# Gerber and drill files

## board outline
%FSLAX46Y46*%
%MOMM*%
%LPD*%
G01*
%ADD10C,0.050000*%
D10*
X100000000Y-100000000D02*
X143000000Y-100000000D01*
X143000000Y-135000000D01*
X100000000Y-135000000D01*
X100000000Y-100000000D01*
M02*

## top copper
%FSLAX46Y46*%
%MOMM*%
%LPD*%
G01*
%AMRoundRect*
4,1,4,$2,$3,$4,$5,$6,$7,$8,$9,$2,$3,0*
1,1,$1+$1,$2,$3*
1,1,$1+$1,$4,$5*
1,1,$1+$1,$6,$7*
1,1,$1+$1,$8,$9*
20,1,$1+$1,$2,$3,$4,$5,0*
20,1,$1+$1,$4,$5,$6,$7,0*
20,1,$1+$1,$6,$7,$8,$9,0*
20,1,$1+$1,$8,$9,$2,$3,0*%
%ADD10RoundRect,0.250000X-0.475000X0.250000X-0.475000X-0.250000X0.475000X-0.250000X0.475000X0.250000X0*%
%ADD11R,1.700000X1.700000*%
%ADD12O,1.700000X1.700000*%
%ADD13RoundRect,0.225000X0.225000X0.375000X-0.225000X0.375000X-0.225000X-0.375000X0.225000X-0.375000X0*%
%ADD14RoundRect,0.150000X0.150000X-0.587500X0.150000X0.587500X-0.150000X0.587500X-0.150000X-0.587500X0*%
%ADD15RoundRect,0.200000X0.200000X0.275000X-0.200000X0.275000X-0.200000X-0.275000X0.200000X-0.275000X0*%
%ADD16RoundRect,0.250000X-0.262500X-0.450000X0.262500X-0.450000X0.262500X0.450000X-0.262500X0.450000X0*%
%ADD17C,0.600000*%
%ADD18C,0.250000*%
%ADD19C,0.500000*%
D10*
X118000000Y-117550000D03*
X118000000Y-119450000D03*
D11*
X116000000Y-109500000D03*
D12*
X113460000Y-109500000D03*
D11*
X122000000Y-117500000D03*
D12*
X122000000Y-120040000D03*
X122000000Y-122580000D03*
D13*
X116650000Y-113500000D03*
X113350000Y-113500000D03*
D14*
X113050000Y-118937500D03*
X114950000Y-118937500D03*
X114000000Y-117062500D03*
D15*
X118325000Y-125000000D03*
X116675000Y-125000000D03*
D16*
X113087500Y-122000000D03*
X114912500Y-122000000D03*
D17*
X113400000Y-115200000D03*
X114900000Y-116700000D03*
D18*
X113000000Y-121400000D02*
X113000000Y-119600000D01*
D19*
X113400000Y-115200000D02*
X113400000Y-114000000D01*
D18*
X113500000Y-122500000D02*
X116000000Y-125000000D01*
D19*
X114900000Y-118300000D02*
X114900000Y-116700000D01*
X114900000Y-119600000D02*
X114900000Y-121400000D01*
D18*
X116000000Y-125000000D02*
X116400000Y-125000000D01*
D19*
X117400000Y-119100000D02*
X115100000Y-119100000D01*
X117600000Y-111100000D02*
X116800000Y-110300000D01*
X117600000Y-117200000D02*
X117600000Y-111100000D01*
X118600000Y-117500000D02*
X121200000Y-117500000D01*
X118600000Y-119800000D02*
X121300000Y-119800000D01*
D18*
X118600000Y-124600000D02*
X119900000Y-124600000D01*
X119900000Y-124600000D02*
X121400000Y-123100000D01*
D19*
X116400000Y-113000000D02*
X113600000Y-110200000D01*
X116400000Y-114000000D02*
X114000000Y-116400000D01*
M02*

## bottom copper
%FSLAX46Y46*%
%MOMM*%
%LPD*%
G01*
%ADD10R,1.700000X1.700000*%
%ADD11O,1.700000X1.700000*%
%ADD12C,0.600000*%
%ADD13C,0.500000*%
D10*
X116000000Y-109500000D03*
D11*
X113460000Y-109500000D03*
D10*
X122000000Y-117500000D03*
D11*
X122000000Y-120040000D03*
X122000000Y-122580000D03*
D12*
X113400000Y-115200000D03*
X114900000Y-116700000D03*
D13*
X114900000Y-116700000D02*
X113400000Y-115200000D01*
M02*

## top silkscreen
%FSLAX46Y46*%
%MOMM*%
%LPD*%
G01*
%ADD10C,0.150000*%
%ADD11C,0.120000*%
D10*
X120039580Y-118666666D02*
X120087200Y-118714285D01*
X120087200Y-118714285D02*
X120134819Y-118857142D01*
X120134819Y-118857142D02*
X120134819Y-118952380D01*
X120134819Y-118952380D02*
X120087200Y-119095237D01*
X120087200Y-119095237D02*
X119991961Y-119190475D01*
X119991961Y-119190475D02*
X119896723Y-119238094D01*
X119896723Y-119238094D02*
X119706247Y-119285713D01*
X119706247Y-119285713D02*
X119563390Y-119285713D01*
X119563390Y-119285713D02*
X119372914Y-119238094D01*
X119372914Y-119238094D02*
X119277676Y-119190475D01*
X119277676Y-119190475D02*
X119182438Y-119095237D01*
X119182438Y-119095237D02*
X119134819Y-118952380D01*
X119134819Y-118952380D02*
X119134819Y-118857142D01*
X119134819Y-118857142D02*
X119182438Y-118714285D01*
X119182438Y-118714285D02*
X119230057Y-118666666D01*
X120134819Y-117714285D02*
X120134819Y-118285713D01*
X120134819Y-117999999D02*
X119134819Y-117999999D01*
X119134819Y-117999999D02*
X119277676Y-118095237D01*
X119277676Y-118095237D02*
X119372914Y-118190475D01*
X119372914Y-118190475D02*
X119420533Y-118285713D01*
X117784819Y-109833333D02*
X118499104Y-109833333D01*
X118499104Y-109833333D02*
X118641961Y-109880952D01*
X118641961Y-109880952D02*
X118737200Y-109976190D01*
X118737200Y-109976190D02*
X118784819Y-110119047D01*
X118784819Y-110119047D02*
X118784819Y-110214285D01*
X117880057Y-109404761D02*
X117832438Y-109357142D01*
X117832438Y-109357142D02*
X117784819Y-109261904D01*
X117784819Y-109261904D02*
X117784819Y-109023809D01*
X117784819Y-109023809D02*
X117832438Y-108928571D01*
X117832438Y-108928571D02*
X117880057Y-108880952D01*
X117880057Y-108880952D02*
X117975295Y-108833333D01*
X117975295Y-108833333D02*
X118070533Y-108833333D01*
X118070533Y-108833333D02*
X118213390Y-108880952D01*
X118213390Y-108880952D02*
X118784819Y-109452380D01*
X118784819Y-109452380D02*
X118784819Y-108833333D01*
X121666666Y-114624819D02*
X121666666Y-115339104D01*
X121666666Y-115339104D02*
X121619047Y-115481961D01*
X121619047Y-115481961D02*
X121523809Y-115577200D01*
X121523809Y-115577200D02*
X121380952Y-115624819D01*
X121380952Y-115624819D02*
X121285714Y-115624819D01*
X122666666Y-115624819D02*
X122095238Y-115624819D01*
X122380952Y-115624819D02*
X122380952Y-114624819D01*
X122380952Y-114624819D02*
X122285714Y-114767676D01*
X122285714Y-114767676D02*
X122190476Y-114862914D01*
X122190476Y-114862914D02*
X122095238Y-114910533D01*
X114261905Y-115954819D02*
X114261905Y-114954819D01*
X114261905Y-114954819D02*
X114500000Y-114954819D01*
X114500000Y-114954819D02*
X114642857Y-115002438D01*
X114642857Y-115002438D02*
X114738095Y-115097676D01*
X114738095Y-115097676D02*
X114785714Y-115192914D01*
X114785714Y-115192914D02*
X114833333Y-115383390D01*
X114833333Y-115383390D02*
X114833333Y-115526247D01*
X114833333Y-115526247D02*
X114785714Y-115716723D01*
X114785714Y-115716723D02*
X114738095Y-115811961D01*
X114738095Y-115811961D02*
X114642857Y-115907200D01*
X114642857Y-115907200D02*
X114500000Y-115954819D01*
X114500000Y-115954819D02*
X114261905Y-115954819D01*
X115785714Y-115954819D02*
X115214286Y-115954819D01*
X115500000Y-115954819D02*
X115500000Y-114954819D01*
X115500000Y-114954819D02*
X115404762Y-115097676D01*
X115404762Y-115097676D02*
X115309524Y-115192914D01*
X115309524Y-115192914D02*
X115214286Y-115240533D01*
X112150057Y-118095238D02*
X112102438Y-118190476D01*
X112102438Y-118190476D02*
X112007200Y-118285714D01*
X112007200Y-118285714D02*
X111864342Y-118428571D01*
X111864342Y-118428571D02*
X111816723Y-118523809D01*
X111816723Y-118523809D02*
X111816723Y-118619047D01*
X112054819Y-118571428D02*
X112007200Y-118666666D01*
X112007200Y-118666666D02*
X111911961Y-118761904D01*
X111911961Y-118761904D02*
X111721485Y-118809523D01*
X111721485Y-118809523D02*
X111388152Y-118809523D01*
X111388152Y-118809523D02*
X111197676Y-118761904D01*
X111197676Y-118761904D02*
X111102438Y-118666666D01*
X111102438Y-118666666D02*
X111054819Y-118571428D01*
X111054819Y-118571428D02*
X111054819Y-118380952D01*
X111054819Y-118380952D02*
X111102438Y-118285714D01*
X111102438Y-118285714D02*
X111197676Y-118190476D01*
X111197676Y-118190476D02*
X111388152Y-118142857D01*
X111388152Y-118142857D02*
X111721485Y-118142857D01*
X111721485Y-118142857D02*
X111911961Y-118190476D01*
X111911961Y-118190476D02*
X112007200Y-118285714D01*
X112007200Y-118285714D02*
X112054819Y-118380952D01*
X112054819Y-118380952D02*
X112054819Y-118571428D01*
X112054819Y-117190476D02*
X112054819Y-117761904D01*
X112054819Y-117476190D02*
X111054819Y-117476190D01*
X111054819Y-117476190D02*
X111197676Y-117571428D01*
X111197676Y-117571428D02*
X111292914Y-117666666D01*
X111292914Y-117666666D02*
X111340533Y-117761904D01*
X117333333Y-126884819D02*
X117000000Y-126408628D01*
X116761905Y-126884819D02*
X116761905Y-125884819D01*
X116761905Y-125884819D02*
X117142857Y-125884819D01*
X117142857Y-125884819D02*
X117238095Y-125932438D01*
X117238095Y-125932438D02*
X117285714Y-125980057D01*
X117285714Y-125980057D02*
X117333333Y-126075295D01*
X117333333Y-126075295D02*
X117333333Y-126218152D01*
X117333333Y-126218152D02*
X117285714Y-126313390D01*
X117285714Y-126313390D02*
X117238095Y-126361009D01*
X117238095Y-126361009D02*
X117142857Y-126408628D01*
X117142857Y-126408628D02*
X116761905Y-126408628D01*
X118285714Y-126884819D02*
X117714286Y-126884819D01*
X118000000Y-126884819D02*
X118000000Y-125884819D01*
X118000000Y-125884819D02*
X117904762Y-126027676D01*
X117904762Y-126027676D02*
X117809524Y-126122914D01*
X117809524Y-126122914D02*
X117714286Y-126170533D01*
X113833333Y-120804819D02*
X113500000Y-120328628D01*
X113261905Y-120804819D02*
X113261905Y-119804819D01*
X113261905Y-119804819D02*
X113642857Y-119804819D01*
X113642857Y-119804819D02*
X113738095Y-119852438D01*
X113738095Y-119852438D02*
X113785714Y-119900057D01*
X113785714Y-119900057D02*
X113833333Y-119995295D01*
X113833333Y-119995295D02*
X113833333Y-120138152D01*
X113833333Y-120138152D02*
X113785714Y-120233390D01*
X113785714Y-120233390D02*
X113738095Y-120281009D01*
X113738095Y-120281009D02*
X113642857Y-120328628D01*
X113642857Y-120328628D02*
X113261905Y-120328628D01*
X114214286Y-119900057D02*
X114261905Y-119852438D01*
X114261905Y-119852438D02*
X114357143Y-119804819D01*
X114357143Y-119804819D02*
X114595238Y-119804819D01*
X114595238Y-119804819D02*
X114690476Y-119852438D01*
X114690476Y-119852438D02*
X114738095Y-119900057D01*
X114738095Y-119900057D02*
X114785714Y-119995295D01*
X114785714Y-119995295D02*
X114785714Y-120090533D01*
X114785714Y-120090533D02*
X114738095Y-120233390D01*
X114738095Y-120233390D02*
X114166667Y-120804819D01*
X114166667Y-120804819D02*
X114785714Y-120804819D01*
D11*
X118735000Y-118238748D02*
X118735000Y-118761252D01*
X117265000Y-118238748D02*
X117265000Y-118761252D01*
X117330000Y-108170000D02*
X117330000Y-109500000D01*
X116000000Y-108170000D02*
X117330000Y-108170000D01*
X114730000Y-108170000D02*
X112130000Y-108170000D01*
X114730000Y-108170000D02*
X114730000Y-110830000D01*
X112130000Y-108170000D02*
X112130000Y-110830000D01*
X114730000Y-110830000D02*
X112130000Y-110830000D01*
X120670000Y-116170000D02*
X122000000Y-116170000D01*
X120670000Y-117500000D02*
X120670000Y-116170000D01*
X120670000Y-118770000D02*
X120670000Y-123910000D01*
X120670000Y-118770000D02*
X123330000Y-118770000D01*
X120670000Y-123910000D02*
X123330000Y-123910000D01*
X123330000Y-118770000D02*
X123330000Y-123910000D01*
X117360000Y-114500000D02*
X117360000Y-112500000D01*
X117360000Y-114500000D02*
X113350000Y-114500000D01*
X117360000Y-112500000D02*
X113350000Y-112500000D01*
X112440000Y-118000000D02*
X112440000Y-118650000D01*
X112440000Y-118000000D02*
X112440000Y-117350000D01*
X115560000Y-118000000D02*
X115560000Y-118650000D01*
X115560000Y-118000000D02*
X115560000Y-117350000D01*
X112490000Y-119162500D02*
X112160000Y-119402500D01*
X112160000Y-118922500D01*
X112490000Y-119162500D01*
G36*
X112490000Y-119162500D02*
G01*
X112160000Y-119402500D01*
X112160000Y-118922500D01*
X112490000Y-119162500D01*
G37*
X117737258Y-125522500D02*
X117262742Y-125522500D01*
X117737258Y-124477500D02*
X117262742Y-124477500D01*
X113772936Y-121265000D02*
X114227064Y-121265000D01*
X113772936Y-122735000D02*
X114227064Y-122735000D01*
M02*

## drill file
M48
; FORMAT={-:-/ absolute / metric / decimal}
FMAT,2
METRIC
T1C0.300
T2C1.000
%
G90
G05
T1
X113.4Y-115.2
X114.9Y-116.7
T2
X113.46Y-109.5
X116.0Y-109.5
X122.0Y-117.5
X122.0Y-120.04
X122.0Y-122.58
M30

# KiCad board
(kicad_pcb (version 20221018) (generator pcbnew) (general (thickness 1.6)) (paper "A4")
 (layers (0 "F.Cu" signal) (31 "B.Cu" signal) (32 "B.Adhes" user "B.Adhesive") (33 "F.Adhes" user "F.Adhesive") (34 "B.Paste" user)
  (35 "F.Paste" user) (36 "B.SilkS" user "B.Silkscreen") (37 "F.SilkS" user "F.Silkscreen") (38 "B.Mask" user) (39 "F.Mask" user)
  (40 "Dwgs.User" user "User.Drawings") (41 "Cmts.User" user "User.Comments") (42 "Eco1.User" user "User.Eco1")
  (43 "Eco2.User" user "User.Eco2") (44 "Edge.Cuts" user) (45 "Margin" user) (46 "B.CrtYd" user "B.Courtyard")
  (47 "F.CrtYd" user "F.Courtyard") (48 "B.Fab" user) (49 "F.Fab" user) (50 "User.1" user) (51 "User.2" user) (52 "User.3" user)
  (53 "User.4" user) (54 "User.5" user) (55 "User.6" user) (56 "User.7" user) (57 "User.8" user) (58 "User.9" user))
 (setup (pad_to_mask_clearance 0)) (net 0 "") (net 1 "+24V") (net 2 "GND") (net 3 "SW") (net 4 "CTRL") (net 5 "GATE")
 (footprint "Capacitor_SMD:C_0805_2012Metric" (layer "F.Cu") (at 118 118.5 -90)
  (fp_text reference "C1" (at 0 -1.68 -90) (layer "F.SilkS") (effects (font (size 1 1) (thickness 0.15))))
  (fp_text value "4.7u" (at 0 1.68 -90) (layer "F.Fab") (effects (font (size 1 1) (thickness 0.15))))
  (fp_line (start -0.261252 -0.735) (end 0.261252 -0.735) (stroke (width 0.12) (type solid)) (layer "F.SilkS"))
  (fp_line (start -0.261252 0.735) (end 0.261252 0.735) (stroke (width 0.12) (type solid)) (layer "F.SilkS"))
  (pad "1" smd roundrect (at -0.95 0 270) (size 1 1.45) (layers "F.Cu" "F.Paste" "F.Mask") (roundrect_rratio 0.25) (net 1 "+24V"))
  (pad "2" smd roundrect (at 0.95 0 270) (size 1 1.45) (layers "F.Cu" "F.Paste" "F.Mask") (roundrect_rratio 0.25) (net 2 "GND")))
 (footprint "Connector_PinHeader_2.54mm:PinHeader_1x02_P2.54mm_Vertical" (layer "F.Cu") (at 116 109.5 -90)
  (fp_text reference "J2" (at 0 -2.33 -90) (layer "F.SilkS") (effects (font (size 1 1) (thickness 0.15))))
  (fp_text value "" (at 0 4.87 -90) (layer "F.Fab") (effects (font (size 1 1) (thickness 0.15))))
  (fp_line (start -1.33 -1.33) (end 0 -1.33) (stroke (width 0.12) (type solid)) (layer "F.SilkS"))
  (fp_line (start -1.33 0) (end -1.33 -1.33) (stroke (width 0.12) (type solid)) (layer "F.SilkS"))
  (fp_line (start -1.33 1.27) (end -1.33 3.87) (stroke (width 0.12) (type solid)) (layer "F.SilkS"))
  (fp_line (start -1.33 1.27) (end 1.33 1.27) (stroke (width 0.12) (type solid)) (layer "F.SilkS"))
  (fp_line (start -1.33 3.87) (end 1.33 3.87) (stroke (width 0.12) (type solid)) (layer "F.SilkS"))
  (fp_line (start 1.33 1.27) (end 1.33 3.87) (stroke (width 0.12) (type solid)) (layer "F.SilkS"))
  (pad "1" thru_hole rect (at 0 0 270) (size 1.7 1.7) (drill 1) (layers "*.Cu" "*.Mask") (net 1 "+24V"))
  (pad "2" thru_hole oval (at 0 2.54 270) (size 1.7 1.7) (drill 1) (layers "*.Cu" "*.Mask") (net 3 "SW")))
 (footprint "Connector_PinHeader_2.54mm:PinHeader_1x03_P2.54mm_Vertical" (layer "F.Cu") (at 122 117.5)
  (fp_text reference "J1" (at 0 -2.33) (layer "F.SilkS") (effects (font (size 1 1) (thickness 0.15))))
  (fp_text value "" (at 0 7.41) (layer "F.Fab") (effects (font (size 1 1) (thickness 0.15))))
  (fp_line (start -1.33 -1.33) (end 0 -1.33) (stroke (width 0.12) (type solid)) (layer "F.SilkS"))
  (fp_line (start -1.33 0) (end -1.33 -1.33) (stroke (width 0.12) (type solid)) (layer "F.SilkS"))
  (fp_line (start -1.33 1.27) (end -1.33 6.41) (stroke (width 0.12) (type solid)) (layer "F.SilkS"))
  (fp_line (start -1.33 1.27) (end 1.33 1.27) (stroke (width 0.12) (type solid)) (layer "F.SilkS"))
  (fp_line (start -1.33 6.41) (end 1.33 6.41) (stroke (width 0.12) (type solid)) (layer "F.SilkS"))
  (fp_line (start 1.33 1.27) (end 1.33 6.41) (stroke (width 0.12) (type solid)) (layer "F.SilkS"))
  (pad "1" thru_hole rect (at 0 0) (size 1.7 1.7) (drill 1) (layers "*.Cu" "*.Mask") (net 1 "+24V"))
  (pad "2" thru_hole oval (at 0 2.54) (size 1.7 1.7) (drill 1) (layers "*.Cu" "*.Mask") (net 2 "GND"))
  (pad "3" thru_hole oval (at 0 5.08) (size 1.7 1.7) (drill 1) (layers "*.Cu" "*.Mask") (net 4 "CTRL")))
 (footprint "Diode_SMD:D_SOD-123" (layer "F.Cu") (at 115 113.5 180)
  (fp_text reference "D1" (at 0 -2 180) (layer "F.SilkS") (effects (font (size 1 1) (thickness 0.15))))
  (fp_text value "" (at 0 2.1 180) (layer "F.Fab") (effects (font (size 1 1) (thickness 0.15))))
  (fp_line (start -2.36 -1) (end -2.36 1) (stroke (width 0.12) (type solid)) (layer "F.SilkS"))
  (fp_line (start -2.36 -1) (end 1.65 -1) (stroke (width 0.12) (type solid)) (layer "F.SilkS"))
  (fp_line (start -2.36 1) (end 1.65 1) (stroke (width 0.12) (type solid)) (layer "F.SilkS"))
  (pad "1" smd roundrect (at -1.65 0 180) (size 0.9 1.2) (layers "F.Cu" "F.Paste" "F.Mask") (roundrect_rratio 0.25) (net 3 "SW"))
  (pad "2" smd roundrect (at 1.65 0 180) (size 0.9 1.2) (layers "F.Cu" "F.Paste" "F.Mask") (roundrect_rratio 0.25) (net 2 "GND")))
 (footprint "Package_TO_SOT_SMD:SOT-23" (layer "F.Cu") (at 114 118 90)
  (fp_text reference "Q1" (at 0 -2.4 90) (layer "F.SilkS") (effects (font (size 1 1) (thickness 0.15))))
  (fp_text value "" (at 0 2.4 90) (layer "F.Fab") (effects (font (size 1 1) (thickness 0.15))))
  (fp_line (start 0 -1.56) (end -0.65 -1.56) (stroke (width 0.12) (type solid)) (layer "F.SilkS"))
  (fp_line (start 0 -1.56) (end 0.65 -1.56) (stroke (width 0.12) (type solid)) (layer "F.SilkS"))
  (fp_line (start 0 1.56) (end -0.65 1.56) (stroke (width 0.12) (type solid)) (layer "F.SilkS"))
  (fp_line (start 0 1.56) (end 0.65 1.56) (stroke (width 0.12) (type solid)) (layer "F.SilkS"))
  (fp_poly
   (pts (xy -1.1625 -1.51) (xy -1.4025 -1.84) (xy -0.9225 -1.84) (xy -1.1625 -1.51)) (stroke (width 0.12) (type solid)) (fill solid)
   (layer "F.SilkS"))
  (pad "1" smd roundrect (at -0.9375 -0.95 90) (size 1.475 0.6) (layers "F.Cu" "F.Paste" "F.Mask") (roundrect_rratio 0.25) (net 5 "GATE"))
  (pad "2" smd roundrect (at -0.9375 0.95 90) (size 1.475 0.6) (layers "F.Cu" "F.Paste" "F.Mask") (roundrect_rratio 0.25) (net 2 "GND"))
  (pad "3" smd roundrect (at 0.9375 0 90) (size 1.475 0.6) (layers "F.Cu" "F.Paste" "F.Mask") (roundrect_rratio 0.25) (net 3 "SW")))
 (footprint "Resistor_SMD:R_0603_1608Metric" (layer "F.Cu") (at 117.5 125 180)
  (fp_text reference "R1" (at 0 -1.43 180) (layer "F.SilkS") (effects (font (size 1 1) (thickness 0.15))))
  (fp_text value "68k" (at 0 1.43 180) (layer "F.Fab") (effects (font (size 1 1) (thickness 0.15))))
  (fp_line (start -0.237258 -0.5225) (end 0.237258 -0.5225) (stroke (width 0.12) (type solid)) (layer "F.SilkS"))
  (fp_line (start -0.237258 0.5225) (end 0.237258 0.5225) (stroke (width 0.12) (type solid)) (layer "F.SilkS"))
  (pad "1" smd roundrect (at -0.825 0 180) (size 0.8 0.95) (layers "F.Cu" "F.Paste" "F.Mask") (roundrect_rratio 0.25) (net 4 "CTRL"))
  (pad "2" smd roundrect (at 0.825 0 180) (size 0.8 0.95) (layers "F.Cu" "F.Paste" "F.Mask") (roundrect_rratio 0.25) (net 5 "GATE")))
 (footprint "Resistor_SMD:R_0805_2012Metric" (layer "F.Cu") (at 114 122)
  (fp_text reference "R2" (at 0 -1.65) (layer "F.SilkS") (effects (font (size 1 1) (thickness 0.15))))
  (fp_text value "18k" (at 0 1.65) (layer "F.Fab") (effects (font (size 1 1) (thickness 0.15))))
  (fp_line (start -0.227064 -0.735) (end 0.227064 -0.735) (stroke (width 0.12) (type solid)) (layer "F.SilkS"))
  (fp_line (start -0.227064 0.735) (end 0.227064 0.735) (stroke (width 0.12) (type solid)) (layer "F.SilkS"))
  (pad "1" smd roundrect (at -0.9125 0) (size 1.025 1.4) (layers "F.Cu" "F.Paste" "F.Mask") (roundrect_rratio 0.243902) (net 5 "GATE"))
  (pad "2" smd roundrect (at 0.9125 0) (size 1.025 1.4) (layers "F.Cu" "F.Paste" "F.Mask") (roundrect_rratio 0.243902) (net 2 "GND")))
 (gr_rect (start 100 100) (end 143 135) (stroke (width 0.05) (type default)) (fill none) (layer "Edge.Cuts"))
 (segment (start 113 121.4) (end 113 119.6) (width 0.25) (layer "F.Cu") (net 5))
 (segment (start 113.4 115.2) (end 113.4 114) (width 0.5) (layer "F.Cu") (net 2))
 (segment (start 113.5 122.5) (end 116 125) (width 0.25) (layer "F.Cu") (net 5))
 (segment (start 114.9 118.3) (end 114.9 116.7) (width 0.5) (layer "F.Cu") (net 2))
 (segment (start 114.9 119.6) (end 114.9 121.4) (width 0.5) (layer "F.Cu") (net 2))
 (segment (start 116 125) (end 116.4 125) (width 0.25) (layer "F.Cu") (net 5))
 (segment (start 117.4 119.1) (end 115.1 119.1) (width 0.5) (layer "F.Cu") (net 2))
 (segment (start 117.6 111.1) (end 116.8 110.3) (width 0.5) (layer "F.Cu") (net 1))
 (segment (start 117.6 117.2) (end 117.6 111.1) (width 0.5) (layer "F.Cu") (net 1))
 (segment (start 118.6 117.5) (end 121.2 117.5) (width 0.5) (layer "F.Cu") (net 1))
 (segment (start 118.6 119.8) (end 121.3 119.8) (width 0.5) (layer "F.Cu") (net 2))
 (segment (start 118.6 124.6) (end 119.9 124.6) (width 0.25) (layer "F.Cu") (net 4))
 (segment (start 119.9 124.6) (end 121.4 123.1) (width 0.25) (layer "F.Cu") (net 4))
 (via (at 113.4 115.2) (size 0.6) (drill 0.3) (layers "F.Cu" "B.Cu") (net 2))
 (via (at 114.9 116.7) (size 0.6) (drill 0.3) (layers "F.Cu" "B.Cu") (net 2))
 (segment (start 114.9 116.7) (end 113.4 115.2) (width 0.5) (layer "B.Cu") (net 2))
 (segment (start 116.4 113) (end 113.6 110.2) (width 0.5) (layer "F.Cu") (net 3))
 (segment (start 116.4 114) (end 114 116.4) (width 0.5) (layer "F.Cu") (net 3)))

